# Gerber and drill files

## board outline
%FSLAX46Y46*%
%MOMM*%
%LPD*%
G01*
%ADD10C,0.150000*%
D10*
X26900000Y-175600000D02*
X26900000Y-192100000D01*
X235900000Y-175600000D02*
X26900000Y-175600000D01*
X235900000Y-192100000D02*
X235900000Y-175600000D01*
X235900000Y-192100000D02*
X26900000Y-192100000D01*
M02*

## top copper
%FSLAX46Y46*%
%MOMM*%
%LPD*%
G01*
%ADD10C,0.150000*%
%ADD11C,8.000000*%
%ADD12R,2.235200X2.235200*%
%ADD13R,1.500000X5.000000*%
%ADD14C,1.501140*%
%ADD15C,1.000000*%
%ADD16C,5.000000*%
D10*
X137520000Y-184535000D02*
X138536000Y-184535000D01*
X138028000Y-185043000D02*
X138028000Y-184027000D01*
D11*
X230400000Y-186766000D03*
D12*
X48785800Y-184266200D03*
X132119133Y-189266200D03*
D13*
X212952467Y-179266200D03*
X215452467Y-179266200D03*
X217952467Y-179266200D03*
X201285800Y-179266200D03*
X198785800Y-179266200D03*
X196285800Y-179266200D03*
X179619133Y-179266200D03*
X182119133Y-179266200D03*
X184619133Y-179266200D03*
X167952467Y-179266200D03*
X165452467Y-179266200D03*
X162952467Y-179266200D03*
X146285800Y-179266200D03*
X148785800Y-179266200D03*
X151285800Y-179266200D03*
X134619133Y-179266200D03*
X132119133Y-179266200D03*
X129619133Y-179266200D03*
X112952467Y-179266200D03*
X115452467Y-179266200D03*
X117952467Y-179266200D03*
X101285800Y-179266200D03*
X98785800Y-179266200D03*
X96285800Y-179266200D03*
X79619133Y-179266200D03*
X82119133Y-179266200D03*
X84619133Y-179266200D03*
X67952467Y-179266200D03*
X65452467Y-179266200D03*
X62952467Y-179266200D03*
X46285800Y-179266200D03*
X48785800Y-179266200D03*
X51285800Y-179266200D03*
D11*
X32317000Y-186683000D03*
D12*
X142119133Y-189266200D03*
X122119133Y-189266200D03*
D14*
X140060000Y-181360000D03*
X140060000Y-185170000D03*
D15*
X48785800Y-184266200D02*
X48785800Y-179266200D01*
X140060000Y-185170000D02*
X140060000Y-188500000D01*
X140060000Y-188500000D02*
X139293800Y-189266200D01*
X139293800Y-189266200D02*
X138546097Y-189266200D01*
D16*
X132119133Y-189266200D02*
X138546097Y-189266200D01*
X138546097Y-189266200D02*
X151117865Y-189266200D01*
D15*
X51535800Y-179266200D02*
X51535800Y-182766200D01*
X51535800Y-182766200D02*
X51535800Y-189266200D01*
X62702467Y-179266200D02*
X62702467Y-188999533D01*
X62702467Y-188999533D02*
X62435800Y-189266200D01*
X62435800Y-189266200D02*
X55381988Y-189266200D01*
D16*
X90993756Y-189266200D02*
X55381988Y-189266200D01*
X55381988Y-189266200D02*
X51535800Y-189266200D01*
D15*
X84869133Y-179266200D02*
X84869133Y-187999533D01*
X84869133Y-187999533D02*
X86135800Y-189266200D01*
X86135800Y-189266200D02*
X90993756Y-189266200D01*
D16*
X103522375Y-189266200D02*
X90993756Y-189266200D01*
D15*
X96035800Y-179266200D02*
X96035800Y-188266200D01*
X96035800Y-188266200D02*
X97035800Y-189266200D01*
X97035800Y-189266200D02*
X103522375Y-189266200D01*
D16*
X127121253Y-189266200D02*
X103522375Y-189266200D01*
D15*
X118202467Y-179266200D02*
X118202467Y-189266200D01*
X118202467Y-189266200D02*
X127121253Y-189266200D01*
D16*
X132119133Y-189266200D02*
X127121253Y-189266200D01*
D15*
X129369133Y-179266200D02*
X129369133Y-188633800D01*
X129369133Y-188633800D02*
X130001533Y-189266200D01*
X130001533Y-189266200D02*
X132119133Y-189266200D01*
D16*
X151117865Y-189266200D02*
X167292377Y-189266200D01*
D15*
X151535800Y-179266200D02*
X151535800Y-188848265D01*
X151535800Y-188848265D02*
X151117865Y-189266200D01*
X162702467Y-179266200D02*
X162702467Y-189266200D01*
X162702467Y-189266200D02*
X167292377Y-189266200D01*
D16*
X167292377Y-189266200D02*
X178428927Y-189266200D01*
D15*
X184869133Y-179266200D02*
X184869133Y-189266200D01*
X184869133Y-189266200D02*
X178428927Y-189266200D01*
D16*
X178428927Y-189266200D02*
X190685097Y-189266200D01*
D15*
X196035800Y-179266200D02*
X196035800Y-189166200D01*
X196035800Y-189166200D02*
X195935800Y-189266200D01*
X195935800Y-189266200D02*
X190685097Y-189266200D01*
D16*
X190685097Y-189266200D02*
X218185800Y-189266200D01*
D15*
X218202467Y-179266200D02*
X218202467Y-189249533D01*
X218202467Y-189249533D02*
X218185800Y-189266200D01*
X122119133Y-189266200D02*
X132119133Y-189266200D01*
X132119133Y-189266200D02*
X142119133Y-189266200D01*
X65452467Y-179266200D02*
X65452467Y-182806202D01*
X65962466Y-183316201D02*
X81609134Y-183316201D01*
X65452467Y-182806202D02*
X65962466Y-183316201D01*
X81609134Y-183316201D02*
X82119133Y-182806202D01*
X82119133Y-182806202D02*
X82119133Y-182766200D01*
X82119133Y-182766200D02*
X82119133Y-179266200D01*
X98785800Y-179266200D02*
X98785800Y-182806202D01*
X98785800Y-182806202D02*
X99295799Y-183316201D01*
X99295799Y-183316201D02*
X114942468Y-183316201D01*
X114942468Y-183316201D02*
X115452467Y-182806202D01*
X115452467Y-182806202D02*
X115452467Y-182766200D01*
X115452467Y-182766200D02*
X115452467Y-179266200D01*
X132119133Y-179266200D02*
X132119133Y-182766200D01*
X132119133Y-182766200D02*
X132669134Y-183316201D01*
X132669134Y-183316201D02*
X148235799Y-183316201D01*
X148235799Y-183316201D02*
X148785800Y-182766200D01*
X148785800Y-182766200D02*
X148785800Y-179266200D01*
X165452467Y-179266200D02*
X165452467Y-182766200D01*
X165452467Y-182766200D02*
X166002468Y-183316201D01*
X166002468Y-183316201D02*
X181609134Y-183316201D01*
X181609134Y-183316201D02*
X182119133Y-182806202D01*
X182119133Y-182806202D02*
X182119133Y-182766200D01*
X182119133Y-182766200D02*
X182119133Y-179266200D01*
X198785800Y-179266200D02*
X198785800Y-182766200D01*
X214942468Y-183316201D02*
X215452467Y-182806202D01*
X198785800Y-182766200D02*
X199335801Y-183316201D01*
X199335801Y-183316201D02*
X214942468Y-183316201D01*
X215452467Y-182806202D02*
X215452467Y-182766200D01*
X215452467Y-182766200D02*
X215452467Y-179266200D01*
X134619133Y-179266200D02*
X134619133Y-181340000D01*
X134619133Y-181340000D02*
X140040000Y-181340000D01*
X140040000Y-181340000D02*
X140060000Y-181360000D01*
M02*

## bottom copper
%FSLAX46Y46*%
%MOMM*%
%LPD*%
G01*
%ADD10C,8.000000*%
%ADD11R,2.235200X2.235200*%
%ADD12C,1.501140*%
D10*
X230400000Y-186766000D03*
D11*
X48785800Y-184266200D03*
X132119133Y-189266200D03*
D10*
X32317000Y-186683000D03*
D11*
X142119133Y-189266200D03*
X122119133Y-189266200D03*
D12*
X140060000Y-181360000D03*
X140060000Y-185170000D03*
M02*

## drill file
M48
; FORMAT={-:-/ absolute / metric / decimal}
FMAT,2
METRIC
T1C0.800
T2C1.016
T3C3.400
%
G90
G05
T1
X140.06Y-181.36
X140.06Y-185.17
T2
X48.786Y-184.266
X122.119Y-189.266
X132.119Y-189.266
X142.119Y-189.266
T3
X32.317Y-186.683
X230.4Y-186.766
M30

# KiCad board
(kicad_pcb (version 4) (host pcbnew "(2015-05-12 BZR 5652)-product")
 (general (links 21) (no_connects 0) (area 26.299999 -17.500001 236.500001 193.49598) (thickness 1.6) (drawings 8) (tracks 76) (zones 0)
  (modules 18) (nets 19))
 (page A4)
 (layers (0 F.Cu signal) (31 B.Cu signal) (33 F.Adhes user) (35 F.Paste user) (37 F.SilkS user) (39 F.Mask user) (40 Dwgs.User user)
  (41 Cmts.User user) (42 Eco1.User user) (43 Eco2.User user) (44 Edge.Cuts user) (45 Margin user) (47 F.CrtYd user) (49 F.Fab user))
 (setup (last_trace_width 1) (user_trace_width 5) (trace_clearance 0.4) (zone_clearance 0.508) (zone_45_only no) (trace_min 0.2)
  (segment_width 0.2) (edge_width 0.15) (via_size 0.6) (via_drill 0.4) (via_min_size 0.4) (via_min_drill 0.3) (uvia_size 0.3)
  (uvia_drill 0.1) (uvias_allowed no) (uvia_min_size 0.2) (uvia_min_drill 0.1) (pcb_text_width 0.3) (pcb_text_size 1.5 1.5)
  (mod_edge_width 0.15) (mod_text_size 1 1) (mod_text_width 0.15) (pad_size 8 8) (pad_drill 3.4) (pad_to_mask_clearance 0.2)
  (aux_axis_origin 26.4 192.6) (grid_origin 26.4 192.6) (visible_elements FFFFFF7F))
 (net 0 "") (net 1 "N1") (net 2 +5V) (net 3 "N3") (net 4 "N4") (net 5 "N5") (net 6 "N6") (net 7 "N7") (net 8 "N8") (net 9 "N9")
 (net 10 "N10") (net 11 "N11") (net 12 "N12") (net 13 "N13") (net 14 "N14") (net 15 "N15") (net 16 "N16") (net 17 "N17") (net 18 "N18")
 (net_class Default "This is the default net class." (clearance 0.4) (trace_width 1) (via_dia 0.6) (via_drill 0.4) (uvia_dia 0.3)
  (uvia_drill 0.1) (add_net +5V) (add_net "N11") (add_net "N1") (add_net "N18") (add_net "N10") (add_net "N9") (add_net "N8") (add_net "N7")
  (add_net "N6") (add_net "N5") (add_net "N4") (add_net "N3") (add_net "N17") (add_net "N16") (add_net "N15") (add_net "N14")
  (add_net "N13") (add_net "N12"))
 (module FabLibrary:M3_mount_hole (layer F.Cu) (at 230.4 186.766)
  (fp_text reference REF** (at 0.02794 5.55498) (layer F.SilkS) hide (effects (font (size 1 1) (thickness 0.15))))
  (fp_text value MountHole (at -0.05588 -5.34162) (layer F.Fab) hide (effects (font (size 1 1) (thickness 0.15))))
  (pad 1 thru_hole circle (at 0 0) (size 8 8) (drill 3.4) (layers *.Cu *.Mask F.SilkS)))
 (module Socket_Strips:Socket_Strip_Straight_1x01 (layer F.Cu) (at 48.7858 184.2662 90)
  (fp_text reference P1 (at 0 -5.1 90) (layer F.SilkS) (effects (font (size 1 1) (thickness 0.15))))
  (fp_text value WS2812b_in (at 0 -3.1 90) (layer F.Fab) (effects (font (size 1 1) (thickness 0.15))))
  (pad 1 thru_hole rect (at 0 0 90) (size 2.2352 2.2352) (drill 1.016) (layers *.Cu *.Mask F.SilkS) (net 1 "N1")))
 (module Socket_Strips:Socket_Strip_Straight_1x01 (layer F.Cu) (at 132.119133 189.2662 90)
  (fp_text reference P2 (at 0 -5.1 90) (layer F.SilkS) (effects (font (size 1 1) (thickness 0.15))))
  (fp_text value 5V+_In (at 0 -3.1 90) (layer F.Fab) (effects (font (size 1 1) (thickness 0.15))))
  (pad 1 thru_hole rect (at 0 0 90) (size 2.2352 2.2352) (drill 1.016) (layers *.Cu *.Mask F.SilkS) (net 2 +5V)))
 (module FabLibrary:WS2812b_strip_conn (layer F.Cu) (at 215.452467 179.2662 270)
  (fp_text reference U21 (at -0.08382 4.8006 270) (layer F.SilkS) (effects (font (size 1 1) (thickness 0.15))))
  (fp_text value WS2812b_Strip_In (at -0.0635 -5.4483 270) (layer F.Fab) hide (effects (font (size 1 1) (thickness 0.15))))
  (pad 1 smd rect (at 0 2.5 270) (size 5 1.5) (layers F.Cu F.Paste F.Mask) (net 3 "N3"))
  (pad 2 smd rect (at 0 0 270) (size 5 1.5) (layers F.Cu F.Paste F.Mask) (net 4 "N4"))
  (pad 3 smd rect (at 0 -2.5 270) (size 5 1.5) (layers F.Cu F.Paste F.Mask) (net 2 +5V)))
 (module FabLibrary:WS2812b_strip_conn (layer F.Cu) (at 198.7858 179.2662 90)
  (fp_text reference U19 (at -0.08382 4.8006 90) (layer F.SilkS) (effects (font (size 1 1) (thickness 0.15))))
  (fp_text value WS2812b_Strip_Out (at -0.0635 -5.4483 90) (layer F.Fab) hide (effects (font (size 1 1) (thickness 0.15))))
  (pad 1 smd rect (at 0 2.5 90) (size 5 1.5) (layers F.Cu F.Paste F.Mask) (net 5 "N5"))
  (pad 2 smd rect (at 0 0 90) (size 5 1.5) (layers F.Cu F.Paste F.Mask) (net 4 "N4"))
  (pad 3 smd rect (at 0 -2.5 90) (size 5 1.5) (layers F.Cu F.Paste F.Mask) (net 2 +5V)))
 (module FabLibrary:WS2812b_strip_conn (layer F.Cu) (at 182.119133 179.2662 270)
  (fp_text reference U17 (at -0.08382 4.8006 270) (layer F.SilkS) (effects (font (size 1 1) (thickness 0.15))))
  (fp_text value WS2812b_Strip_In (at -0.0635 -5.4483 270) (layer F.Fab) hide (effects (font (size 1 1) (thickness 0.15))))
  (pad 1 smd rect (at 0 2.5 270) (size 5 1.5) (layers F.Cu F.Paste F.Mask) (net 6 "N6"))
  (pad 2 smd rect (at 0 0 270) (size 5 1.5) (layers F.Cu F.Paste F.Mask) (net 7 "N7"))
  (pad 3 smd rect (at 0 -2.5 270) (size 5 1.5) (layers F.Cu F.Paste F.Mask) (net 2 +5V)))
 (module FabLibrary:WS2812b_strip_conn (layer F.Cu) (at 165.452467 179.2662 90)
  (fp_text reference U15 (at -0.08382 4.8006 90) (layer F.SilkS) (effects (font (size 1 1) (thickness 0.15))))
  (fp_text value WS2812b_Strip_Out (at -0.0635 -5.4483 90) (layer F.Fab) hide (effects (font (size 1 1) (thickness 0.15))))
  (pad 1 smd rect (at 0 2.5 90) (size 5 1.5) (layers F.Cu F.Paste F.Mask) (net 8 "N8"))
  (pad 2 smd rect (at 0 0 90) (size 5 1.5) (layers F.Cu F.Paste F.Mask) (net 7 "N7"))
  (pad 3 smd rect (at 0 -2.5 90) (size 5 1.5) (layers F.Cu F.Paste F.Mask) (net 2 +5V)))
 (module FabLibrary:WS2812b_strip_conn (layer F.Cu) (at 148.7858 179.2662 270)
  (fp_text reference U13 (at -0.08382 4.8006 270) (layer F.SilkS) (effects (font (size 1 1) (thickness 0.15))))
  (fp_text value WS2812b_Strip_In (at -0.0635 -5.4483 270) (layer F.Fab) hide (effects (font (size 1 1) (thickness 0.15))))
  (pad 1 smd rect (at 0 2.5 270) (size 5 1.5) (layers F.Cu F.Paste F.Mask) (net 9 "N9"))
  (pad 2 smd rect (at 0 0 270) (size 5 1.5) (layers F.Cu F.Paste F.Mask) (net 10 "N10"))
  (pad 3 smd rect (at 0 -2.5 270) (size 5 1.5) (layers F.Cu F.Paste F.Mask) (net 2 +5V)))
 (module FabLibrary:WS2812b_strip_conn (layer F.Cu) (at 132.119133 179.2662 90)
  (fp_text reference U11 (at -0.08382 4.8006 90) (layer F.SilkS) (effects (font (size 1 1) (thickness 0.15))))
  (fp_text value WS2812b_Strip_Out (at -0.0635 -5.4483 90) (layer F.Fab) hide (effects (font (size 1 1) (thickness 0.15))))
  (pad 1 smd rect (at 0 2.5 90) (size 5 1.5) (layers F.Cu F.Paste F.Mask) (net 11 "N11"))
  (pad 2 smd rect (at 0 0 90) (size 5 1.5) (layers F.Cu F.Paste F.Mask) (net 10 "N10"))
  (pad 3 smd rect (at 0 -2.5 90) (size 5 1.5) (layers F.Cu F.Paste F.Mask) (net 2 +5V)))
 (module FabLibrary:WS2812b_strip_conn (layer F.Cu) (at 115.452467 179.2662 270)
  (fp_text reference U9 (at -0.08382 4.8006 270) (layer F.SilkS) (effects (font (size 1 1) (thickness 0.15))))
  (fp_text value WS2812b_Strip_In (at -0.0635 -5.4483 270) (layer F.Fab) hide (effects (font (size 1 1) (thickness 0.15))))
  (pad 1 smd rect (at 0 2.5 270) (size 5 1.5) (layers F.Cu F.Paste F.Mask) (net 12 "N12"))
  (pad 2 smd rect (at 0 0 270) (size 5 1.5) (layers F.Cu F.Paste F.Mask) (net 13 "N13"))
  (pad 3 smd rect (at 0 -2.5 270) (size 5 1.5) (layers F.Cu F.Paste F.Mask) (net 2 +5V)))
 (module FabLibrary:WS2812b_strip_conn (layer F.Cu) (at 98.7858 179.2662 90)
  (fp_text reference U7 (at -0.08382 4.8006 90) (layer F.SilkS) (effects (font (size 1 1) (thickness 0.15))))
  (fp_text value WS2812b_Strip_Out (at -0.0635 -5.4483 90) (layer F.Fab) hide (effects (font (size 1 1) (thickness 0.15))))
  (pad 1 smd rect (at 0 2.5 90) (size 5 1.5) (layers F.Cu F.Paste F.Mask) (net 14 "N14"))
  (pad 2 smd rect (at 0 0 90) (size 5 1.5) (layers F.Cu F.Paste F.Mask) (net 13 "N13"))
  (pad 3 smd rect (at 0 -2.5 90) (size 5 1.5) (layers F.Cu F.Paste F.Mask) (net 2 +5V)))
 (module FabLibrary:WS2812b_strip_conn (layer F.Cu) (at 82.119133 179.2662 270)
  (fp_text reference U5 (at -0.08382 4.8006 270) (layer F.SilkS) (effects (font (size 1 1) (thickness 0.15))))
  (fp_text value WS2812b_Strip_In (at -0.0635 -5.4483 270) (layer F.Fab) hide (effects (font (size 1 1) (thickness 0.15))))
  (pad 1 smd rect (at 0 2.5 270) (size 5 1.5) (layers F.Cu F.Paste F.Mask) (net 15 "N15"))
  (pad 2 smd rect (at 0 0 270) (size 5 1.5) (layers F.Cu F.Paste F.Mask) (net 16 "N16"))
  (pad 3 smd rect (at 0 -2.5 270) (size 5 1.5) (layers F.Cu F.Paste F.Mask) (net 2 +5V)))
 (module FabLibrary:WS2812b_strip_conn (layer F.Cu) (at 65.452467 179.2662 90)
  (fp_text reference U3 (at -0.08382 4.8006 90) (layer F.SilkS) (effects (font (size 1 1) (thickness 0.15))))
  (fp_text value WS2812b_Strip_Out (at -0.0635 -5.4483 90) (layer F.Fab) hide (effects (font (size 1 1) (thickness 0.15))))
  (pad 1 smd rect (at 0 2.5 90) (size 5 1.5) (layers F.Cu F.Paste F.Mask) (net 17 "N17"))
  (pad 2 smd rect (at 0 0 90) (size 5 1.5) (layers F.Cu F.Paste F.Mask) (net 16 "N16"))
  (pad 3 smd rect (at 0 -2.5 90) (size 5 1.5) (layers F.Cu F.Paste F.Mask) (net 2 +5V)))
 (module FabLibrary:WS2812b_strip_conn (layer F.Cu) (at 48.7858 179.2662 270)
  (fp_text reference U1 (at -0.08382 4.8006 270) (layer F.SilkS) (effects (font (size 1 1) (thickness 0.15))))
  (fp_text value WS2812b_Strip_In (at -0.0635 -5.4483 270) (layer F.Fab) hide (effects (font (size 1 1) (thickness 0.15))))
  (pad 1 smd rect (at 0 2.5 270) (size 5 1.5) (layers F.Cu F.Paste F.Mask) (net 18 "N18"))
  (pad 2 smd rect (at 0 0 270) (size 5 1.5) (layers F.Cu F.Paste F.Mask) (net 1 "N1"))
  (pad 3 smd rect (at 0 -2.5 270) (size 5 1.5) (layers F.Cu F.Paste F.Mask) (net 2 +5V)))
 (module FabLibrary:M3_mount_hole (layer F.Cu) (at 32.317 186.683)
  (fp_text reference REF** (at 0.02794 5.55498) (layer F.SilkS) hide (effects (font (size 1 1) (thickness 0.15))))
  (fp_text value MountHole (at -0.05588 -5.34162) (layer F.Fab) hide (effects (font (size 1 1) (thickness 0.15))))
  (pad 1 thru_hole circle (at 0 0) (size 8 8) (drill 3.4) (layers *.Cu *.Mask F.SilkS)))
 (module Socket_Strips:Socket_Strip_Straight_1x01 (layer F.Cu) (at 142.119133 189.2662)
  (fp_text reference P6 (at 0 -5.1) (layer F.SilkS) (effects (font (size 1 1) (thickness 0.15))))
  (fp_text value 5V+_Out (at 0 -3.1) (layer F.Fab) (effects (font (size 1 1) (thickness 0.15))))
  (pad 1 thru_hole rect (at 0 0) (size 2.2352 2.2352) (drill 1.016) (layers *.Cu *.Mask F.SilkS) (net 2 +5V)))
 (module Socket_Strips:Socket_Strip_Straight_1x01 (layer F.Cu) (at 122.119133 189.2662)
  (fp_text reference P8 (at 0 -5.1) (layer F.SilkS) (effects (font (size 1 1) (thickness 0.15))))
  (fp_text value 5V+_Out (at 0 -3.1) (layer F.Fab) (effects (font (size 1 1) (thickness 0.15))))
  (pad 1 thru_hole rect (at 0 0) (size 2.2352 2.2352) (drill 1.016) (layers *.Cu *.Mask F.SilkS) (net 2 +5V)))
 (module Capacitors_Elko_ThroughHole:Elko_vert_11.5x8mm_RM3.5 (layer F.Cu) (at 140.06 185.17 90)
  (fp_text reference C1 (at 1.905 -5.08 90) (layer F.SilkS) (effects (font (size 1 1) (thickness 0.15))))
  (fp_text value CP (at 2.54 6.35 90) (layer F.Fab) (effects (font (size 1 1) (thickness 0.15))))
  (fp_line (start 0.635 -2.54) (end 0.635 -1.524) (layer F.Cu) (width 0.15))
  (fp_line (start 0.127 -2.032) (end 1.143 -2.032) (layer F.Cu) (width 0.15))
  (pad 2 thru_hole circle (at 3.81 0 90) (size 1.50114 1.50114) (drill 0.8001) (layers *.Cu *.Mask F.SilkS) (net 11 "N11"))
  (pad 1 thru_hole circle (at 0 0 90) (size 1.50114 1.50114) (drill 0.8001) (layers *.Cu *.Mask F.SilkS) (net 2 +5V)))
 (gr_line (start 26.9 175.6) (end 26.9 192.1) (layer Edge.Cuts) (width 0.15))
 (gr_line (start 235.9 175.6) (end 26.9 175.6) (layer Edge.Cuts) (width 0.15))
 (gr_line (start 235.9 192.1) (end 235.9 175.6) (layer Edge.Cuts) (width 0.15))
 (gr_line (start 235.9 192.1) (end 26.9 192.1) (angle 90) (layer Edge.Cuts) (width 0.15))
 (segment (start 48.7858 184.2662) (end 48.7858 179.2662) (width 1) (layer F.Cu) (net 1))
 (segment (start 140.06 185.17) (end 140.06 188.5) (width 1) (layer F.Cu) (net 2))
 (segment (start 140.06 188.5) (end 139.2938 189.2662) (width 1) (layer F.Cu) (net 2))
 (segment (start 139.2938 189.2662) (end 138.546097 189.2662) (width 1) (layer F.Cu) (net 2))
 (segment (start 132.119133 189.2662) (end 138.546097 189.2662) (width 5) (layer F.Cu) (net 2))
 (segment (start 138.546097 189.2662) (end 151.117865 189.2662) (width 5) (layer F.Cu) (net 2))
 (segment (start 51.5358 179.2662) (end 51.5358 182.7662) (width 1) (layer F.Cu) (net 2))
 (segment (start 51.5358 182.7662) (end 51.5358 189.2662) (width 1) (layer F.Cu) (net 2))
 (segment (start 62.702467 179.2662) (end 62.702467 188.999533) (width 1) (layer F.Cu) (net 2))
 (segment (start 62.702467 188.999533) (end 62.4358 189.2662) (width 1) (layer F.Cu) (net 2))
 (segment (start 62.4358 189.2662) (end 55.381988 189.2662) (width 1) (layer F.Cu) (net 2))
 (segment (start 90.993756 189.2662) (end 55.381988 189.2662) (width 5) (layer F.Cu) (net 2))
 (segment (start 55.381988 189.2662) (end 51.5358 189.2662) (width 5) (layer F.Cu) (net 2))
 (segment (start 84.869133 179.2662) (end 84.869133 187.999533) (width 1) (layer F.Cu) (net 2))
 (segment (start 84.869133 187.999533) (end 86.1358 189.2662) (width 1) (layer F.Cu) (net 2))
 (segment (start 86.1358 189.2662) (end 90.993756 189.2662) (width 1) (layer F.Cu) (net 2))
 (segment (start 103.522375 189.2662) (end 90.993756 189.2662) (width 5) (layer F.Cu) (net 2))
 (segment (start 96.0358 179.2662) (end 96.0358 188.2662) (width 1) (layer F.Cu) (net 2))
 (segment (start 96.0358 188.2662) (end 97.0358 189.2662) (width 1) (layer F.Cu) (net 2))
 (segment (start 97.0358 189.2662) (end 103.522375 189.2662) (width 1) (layer F.Cu) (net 2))
 (segment (start 127.121253 189.2662) (end 103.522375 189.2662) (width 5) (layer F.Cu) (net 2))
 (segment (start 118.202467 179.2662) (end 118.202467 189.2662) (width 1) (layer F.Cu) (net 2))
 (segment (start 118.202467 189.2662) (end 127.121253 189.2662) (width 1) (layer F.Cu) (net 2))
 (segment (start 132.119133 189.2662) (end 127.121253 189.2662) (width 5) (layer F.Cu) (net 2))
 (segment (start 129.369133 179.2662) (end 129.369133 188.6338) (width 1) (layer F.Cu) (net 2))
 (segment (start 129.369133 188.6338) (end 130.001533 189.2662) (width 1) (layer F.Cu) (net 2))
 (segment (start 130.001533 189.2662) (end 132.119133 189.2662) (width 1) (layer F.Cu) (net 2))
 (segment (start 151.117865 189.2662) (end 167.292377 189.2662) (width 5) (layer F.Cu) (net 2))
 (segment (start 151.5358 179.2662) (end 151.5358 188.848265) (width 1) (layer F.Cu) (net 2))
 (segment (start 151.5358 188.848265) (end 151.117865 189.2662) (width 1) (layer F.Cu) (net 2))
 (segment (start 162.702467 179.2662) (end 162.702467 189.2662) (width 1) (layer F.Cu) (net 2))
 (segment (start 162.702467 189.2662) (end 167.292377 189.2662) (width 1) (layer F.Cu) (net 2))
 (segment (start 167.292377 189.2662) (end 178.428927 189.2662) (width 5) (layer F.Cu) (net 2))
 (segment (start 184.869133 179.2662) (end 184.869133 189.2662) (width 1) (layer F.Cu) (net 2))
 (segment (start 184.869133 189.2662) (end 178.428927 189.2662) (width 1) (layer F.Cu) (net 2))
 (segment (start 178.428927 189.2662) (end 190.685097 189.2662) (width 5) (layer F.Cu) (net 2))
 (segment (start 196.0358 179.2662) (end 196.0358 189.1662) (width 1) (layer F.Cu) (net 2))
 (segment (start 196.0358 189.1662) (end 195.9358 189.2662) (width 1) (layer F.Cu) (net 2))
 (segment (start 195.9358 189.2662) (end 190.685097 189.2662) (width 1) (layer F.Cu) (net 2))
 (segment (start 190.685097 189.2662) (end 218.1858 189.2662) (width 5) (layer F.Cu) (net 2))
 (segment (start 218.202467 179.2662) (end 218.202467 189.249533) (width 1) (layer F.Cu) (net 2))
 (segment (start 218.202467 189.249533) (end 218.1858 189.2662) (width 1) (layer F.Cu) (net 2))
 (segment (start 122.119133 189.2662) (end 132.119133 189.2662) (width 1) (layer F.Cu) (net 2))
 (segment (start 132.119133 189.2662) (end 142.119133 189.2662) (width 1) (layer F.Cu) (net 2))
 (segment (start 65.452467 179.2662) (end 65.452467 182.806202) (width 1) (layer F.Cu) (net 16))
 (segment (start 65.962466 183.316201) (end 81.609134 183.316201) (width 1) (layer F.Cu) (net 16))
 (segment (start 65.452467 182.806202) (end 65.962466 183.316201) (width 1) (layer F.Cu) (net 16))
 (segment (start 81.609134 183.316201) (end 82.119133 182.806202) (width 1) (layer F.Cu) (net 16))
 (segment (start 82.119133 182.806202) (end 82.119133 182.7662) (width 1) (layer F.Cu) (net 16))
 (segment (start 82.119133 182.7662) (end 82.119133 179.2662) (width 1) (layer F.Cu) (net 16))
 (segment (start 98.7858 179.2662) (end 98.7858 182.806202) (width 1) (layer F.Cu) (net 13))
 (segment (start 98.7858 182.806202) (end 99.295799 183.316201) (width 1) (layer F.Cu) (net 13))
 (segment (start 99.295799 183.316201) (end 114.942468 183.316201) (width 1) (layer F.Cu) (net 13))
 (segment (start 114.942468 183.316201) (end 115.452467 182.806202) (width 1) (layer F.Cu) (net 13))
 (segment (start 115.452467 182.806202) (end 115.452467 182.7662) (width 1) (layer F.Cu) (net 13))
 (segment (start 115.452467 182.7662) (end 115.452467 179.2662) (width 1) (layer F.Cu) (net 13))
 (segment (start 132.119133 179.2662) (end 132.119133 182.7662) (width 1) (layer F.Cu) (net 10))
 (segment (start 132.119133 182.7662) (end 132.669134 183.316201) (width 1) (layer F.Cu) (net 10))
 (segment (start 132.669134 183.316201) (end 148.235799 183.316201) (width 1) (layer F.Cu) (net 10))
 (segment (start 148.235799 183.316201) (end 148.7858 182.7662) (width 1) (layer F.Cu) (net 10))
 (segment (start 148.7858 182.7662) (end 148.7858 179.2662) (width 1) (layer F.Cu) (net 10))
 (segment (start 165.452467 179.2662) (end 165.452467 182.7662) (width 1) (layer F.Cu) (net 7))
 (segment (start 165.452467 182.7662) (end 166.002468 183.316201) (width 1) (layer F.Cu) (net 7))
 (segment (start 166.002468 183.316201) (end 181.609134 183.316201) (width 1) (layer F.Cu) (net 7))
 (segment (start 181.609134 183.316201) (end 182.119133 182.806202) (width 1) (layer F.Cu) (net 7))
 (segment (start 182.119133 182.806202) (end 182.119133 182.7662) (width 1) (layer F.Cu) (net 7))
 (segment (start 182.119133 182.7662) (end 182.119133 179.2662) (width 1) (layer F.Cu) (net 7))
 (segment (start 198.7858 179.2662) (end 198.7858 182.7662) (width 1) (layer F.Cu) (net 4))
 (segment (start 214.942468 183.316201) (end 215.452467 182.806202) (width 1) (layer F.Cu) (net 4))
 (segment (start 198.7858 182.7662) (end 199.335801 183.316201) (width 1) (layer F.Cu) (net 4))
 (segment (start 199.335801 183.316201) (end 214.942468 183.316201) (width 1) (layer F.Cu) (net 4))
 (segment (start 215.452467 182.806202) (end 215.452467 182.7662) (width 1) (layer F.Cu) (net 4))
 (segment (start 215.452467 182.7662) (end 215.452467 179.2662) (width 1) (layer F.Cu) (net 4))
 (segment (start 134.619133 179.2662) (end 134.619133 181.34) (width 1) (layer F.Cu) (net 11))
 (segment (start 134.619133 181.34) (end 140.04 181.34) (width 1) (layer F.Cu) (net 11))
 (segment (start 140.04 181.34) (end 140.06 181.36) (width 1) (layer F.Cu) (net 11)))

